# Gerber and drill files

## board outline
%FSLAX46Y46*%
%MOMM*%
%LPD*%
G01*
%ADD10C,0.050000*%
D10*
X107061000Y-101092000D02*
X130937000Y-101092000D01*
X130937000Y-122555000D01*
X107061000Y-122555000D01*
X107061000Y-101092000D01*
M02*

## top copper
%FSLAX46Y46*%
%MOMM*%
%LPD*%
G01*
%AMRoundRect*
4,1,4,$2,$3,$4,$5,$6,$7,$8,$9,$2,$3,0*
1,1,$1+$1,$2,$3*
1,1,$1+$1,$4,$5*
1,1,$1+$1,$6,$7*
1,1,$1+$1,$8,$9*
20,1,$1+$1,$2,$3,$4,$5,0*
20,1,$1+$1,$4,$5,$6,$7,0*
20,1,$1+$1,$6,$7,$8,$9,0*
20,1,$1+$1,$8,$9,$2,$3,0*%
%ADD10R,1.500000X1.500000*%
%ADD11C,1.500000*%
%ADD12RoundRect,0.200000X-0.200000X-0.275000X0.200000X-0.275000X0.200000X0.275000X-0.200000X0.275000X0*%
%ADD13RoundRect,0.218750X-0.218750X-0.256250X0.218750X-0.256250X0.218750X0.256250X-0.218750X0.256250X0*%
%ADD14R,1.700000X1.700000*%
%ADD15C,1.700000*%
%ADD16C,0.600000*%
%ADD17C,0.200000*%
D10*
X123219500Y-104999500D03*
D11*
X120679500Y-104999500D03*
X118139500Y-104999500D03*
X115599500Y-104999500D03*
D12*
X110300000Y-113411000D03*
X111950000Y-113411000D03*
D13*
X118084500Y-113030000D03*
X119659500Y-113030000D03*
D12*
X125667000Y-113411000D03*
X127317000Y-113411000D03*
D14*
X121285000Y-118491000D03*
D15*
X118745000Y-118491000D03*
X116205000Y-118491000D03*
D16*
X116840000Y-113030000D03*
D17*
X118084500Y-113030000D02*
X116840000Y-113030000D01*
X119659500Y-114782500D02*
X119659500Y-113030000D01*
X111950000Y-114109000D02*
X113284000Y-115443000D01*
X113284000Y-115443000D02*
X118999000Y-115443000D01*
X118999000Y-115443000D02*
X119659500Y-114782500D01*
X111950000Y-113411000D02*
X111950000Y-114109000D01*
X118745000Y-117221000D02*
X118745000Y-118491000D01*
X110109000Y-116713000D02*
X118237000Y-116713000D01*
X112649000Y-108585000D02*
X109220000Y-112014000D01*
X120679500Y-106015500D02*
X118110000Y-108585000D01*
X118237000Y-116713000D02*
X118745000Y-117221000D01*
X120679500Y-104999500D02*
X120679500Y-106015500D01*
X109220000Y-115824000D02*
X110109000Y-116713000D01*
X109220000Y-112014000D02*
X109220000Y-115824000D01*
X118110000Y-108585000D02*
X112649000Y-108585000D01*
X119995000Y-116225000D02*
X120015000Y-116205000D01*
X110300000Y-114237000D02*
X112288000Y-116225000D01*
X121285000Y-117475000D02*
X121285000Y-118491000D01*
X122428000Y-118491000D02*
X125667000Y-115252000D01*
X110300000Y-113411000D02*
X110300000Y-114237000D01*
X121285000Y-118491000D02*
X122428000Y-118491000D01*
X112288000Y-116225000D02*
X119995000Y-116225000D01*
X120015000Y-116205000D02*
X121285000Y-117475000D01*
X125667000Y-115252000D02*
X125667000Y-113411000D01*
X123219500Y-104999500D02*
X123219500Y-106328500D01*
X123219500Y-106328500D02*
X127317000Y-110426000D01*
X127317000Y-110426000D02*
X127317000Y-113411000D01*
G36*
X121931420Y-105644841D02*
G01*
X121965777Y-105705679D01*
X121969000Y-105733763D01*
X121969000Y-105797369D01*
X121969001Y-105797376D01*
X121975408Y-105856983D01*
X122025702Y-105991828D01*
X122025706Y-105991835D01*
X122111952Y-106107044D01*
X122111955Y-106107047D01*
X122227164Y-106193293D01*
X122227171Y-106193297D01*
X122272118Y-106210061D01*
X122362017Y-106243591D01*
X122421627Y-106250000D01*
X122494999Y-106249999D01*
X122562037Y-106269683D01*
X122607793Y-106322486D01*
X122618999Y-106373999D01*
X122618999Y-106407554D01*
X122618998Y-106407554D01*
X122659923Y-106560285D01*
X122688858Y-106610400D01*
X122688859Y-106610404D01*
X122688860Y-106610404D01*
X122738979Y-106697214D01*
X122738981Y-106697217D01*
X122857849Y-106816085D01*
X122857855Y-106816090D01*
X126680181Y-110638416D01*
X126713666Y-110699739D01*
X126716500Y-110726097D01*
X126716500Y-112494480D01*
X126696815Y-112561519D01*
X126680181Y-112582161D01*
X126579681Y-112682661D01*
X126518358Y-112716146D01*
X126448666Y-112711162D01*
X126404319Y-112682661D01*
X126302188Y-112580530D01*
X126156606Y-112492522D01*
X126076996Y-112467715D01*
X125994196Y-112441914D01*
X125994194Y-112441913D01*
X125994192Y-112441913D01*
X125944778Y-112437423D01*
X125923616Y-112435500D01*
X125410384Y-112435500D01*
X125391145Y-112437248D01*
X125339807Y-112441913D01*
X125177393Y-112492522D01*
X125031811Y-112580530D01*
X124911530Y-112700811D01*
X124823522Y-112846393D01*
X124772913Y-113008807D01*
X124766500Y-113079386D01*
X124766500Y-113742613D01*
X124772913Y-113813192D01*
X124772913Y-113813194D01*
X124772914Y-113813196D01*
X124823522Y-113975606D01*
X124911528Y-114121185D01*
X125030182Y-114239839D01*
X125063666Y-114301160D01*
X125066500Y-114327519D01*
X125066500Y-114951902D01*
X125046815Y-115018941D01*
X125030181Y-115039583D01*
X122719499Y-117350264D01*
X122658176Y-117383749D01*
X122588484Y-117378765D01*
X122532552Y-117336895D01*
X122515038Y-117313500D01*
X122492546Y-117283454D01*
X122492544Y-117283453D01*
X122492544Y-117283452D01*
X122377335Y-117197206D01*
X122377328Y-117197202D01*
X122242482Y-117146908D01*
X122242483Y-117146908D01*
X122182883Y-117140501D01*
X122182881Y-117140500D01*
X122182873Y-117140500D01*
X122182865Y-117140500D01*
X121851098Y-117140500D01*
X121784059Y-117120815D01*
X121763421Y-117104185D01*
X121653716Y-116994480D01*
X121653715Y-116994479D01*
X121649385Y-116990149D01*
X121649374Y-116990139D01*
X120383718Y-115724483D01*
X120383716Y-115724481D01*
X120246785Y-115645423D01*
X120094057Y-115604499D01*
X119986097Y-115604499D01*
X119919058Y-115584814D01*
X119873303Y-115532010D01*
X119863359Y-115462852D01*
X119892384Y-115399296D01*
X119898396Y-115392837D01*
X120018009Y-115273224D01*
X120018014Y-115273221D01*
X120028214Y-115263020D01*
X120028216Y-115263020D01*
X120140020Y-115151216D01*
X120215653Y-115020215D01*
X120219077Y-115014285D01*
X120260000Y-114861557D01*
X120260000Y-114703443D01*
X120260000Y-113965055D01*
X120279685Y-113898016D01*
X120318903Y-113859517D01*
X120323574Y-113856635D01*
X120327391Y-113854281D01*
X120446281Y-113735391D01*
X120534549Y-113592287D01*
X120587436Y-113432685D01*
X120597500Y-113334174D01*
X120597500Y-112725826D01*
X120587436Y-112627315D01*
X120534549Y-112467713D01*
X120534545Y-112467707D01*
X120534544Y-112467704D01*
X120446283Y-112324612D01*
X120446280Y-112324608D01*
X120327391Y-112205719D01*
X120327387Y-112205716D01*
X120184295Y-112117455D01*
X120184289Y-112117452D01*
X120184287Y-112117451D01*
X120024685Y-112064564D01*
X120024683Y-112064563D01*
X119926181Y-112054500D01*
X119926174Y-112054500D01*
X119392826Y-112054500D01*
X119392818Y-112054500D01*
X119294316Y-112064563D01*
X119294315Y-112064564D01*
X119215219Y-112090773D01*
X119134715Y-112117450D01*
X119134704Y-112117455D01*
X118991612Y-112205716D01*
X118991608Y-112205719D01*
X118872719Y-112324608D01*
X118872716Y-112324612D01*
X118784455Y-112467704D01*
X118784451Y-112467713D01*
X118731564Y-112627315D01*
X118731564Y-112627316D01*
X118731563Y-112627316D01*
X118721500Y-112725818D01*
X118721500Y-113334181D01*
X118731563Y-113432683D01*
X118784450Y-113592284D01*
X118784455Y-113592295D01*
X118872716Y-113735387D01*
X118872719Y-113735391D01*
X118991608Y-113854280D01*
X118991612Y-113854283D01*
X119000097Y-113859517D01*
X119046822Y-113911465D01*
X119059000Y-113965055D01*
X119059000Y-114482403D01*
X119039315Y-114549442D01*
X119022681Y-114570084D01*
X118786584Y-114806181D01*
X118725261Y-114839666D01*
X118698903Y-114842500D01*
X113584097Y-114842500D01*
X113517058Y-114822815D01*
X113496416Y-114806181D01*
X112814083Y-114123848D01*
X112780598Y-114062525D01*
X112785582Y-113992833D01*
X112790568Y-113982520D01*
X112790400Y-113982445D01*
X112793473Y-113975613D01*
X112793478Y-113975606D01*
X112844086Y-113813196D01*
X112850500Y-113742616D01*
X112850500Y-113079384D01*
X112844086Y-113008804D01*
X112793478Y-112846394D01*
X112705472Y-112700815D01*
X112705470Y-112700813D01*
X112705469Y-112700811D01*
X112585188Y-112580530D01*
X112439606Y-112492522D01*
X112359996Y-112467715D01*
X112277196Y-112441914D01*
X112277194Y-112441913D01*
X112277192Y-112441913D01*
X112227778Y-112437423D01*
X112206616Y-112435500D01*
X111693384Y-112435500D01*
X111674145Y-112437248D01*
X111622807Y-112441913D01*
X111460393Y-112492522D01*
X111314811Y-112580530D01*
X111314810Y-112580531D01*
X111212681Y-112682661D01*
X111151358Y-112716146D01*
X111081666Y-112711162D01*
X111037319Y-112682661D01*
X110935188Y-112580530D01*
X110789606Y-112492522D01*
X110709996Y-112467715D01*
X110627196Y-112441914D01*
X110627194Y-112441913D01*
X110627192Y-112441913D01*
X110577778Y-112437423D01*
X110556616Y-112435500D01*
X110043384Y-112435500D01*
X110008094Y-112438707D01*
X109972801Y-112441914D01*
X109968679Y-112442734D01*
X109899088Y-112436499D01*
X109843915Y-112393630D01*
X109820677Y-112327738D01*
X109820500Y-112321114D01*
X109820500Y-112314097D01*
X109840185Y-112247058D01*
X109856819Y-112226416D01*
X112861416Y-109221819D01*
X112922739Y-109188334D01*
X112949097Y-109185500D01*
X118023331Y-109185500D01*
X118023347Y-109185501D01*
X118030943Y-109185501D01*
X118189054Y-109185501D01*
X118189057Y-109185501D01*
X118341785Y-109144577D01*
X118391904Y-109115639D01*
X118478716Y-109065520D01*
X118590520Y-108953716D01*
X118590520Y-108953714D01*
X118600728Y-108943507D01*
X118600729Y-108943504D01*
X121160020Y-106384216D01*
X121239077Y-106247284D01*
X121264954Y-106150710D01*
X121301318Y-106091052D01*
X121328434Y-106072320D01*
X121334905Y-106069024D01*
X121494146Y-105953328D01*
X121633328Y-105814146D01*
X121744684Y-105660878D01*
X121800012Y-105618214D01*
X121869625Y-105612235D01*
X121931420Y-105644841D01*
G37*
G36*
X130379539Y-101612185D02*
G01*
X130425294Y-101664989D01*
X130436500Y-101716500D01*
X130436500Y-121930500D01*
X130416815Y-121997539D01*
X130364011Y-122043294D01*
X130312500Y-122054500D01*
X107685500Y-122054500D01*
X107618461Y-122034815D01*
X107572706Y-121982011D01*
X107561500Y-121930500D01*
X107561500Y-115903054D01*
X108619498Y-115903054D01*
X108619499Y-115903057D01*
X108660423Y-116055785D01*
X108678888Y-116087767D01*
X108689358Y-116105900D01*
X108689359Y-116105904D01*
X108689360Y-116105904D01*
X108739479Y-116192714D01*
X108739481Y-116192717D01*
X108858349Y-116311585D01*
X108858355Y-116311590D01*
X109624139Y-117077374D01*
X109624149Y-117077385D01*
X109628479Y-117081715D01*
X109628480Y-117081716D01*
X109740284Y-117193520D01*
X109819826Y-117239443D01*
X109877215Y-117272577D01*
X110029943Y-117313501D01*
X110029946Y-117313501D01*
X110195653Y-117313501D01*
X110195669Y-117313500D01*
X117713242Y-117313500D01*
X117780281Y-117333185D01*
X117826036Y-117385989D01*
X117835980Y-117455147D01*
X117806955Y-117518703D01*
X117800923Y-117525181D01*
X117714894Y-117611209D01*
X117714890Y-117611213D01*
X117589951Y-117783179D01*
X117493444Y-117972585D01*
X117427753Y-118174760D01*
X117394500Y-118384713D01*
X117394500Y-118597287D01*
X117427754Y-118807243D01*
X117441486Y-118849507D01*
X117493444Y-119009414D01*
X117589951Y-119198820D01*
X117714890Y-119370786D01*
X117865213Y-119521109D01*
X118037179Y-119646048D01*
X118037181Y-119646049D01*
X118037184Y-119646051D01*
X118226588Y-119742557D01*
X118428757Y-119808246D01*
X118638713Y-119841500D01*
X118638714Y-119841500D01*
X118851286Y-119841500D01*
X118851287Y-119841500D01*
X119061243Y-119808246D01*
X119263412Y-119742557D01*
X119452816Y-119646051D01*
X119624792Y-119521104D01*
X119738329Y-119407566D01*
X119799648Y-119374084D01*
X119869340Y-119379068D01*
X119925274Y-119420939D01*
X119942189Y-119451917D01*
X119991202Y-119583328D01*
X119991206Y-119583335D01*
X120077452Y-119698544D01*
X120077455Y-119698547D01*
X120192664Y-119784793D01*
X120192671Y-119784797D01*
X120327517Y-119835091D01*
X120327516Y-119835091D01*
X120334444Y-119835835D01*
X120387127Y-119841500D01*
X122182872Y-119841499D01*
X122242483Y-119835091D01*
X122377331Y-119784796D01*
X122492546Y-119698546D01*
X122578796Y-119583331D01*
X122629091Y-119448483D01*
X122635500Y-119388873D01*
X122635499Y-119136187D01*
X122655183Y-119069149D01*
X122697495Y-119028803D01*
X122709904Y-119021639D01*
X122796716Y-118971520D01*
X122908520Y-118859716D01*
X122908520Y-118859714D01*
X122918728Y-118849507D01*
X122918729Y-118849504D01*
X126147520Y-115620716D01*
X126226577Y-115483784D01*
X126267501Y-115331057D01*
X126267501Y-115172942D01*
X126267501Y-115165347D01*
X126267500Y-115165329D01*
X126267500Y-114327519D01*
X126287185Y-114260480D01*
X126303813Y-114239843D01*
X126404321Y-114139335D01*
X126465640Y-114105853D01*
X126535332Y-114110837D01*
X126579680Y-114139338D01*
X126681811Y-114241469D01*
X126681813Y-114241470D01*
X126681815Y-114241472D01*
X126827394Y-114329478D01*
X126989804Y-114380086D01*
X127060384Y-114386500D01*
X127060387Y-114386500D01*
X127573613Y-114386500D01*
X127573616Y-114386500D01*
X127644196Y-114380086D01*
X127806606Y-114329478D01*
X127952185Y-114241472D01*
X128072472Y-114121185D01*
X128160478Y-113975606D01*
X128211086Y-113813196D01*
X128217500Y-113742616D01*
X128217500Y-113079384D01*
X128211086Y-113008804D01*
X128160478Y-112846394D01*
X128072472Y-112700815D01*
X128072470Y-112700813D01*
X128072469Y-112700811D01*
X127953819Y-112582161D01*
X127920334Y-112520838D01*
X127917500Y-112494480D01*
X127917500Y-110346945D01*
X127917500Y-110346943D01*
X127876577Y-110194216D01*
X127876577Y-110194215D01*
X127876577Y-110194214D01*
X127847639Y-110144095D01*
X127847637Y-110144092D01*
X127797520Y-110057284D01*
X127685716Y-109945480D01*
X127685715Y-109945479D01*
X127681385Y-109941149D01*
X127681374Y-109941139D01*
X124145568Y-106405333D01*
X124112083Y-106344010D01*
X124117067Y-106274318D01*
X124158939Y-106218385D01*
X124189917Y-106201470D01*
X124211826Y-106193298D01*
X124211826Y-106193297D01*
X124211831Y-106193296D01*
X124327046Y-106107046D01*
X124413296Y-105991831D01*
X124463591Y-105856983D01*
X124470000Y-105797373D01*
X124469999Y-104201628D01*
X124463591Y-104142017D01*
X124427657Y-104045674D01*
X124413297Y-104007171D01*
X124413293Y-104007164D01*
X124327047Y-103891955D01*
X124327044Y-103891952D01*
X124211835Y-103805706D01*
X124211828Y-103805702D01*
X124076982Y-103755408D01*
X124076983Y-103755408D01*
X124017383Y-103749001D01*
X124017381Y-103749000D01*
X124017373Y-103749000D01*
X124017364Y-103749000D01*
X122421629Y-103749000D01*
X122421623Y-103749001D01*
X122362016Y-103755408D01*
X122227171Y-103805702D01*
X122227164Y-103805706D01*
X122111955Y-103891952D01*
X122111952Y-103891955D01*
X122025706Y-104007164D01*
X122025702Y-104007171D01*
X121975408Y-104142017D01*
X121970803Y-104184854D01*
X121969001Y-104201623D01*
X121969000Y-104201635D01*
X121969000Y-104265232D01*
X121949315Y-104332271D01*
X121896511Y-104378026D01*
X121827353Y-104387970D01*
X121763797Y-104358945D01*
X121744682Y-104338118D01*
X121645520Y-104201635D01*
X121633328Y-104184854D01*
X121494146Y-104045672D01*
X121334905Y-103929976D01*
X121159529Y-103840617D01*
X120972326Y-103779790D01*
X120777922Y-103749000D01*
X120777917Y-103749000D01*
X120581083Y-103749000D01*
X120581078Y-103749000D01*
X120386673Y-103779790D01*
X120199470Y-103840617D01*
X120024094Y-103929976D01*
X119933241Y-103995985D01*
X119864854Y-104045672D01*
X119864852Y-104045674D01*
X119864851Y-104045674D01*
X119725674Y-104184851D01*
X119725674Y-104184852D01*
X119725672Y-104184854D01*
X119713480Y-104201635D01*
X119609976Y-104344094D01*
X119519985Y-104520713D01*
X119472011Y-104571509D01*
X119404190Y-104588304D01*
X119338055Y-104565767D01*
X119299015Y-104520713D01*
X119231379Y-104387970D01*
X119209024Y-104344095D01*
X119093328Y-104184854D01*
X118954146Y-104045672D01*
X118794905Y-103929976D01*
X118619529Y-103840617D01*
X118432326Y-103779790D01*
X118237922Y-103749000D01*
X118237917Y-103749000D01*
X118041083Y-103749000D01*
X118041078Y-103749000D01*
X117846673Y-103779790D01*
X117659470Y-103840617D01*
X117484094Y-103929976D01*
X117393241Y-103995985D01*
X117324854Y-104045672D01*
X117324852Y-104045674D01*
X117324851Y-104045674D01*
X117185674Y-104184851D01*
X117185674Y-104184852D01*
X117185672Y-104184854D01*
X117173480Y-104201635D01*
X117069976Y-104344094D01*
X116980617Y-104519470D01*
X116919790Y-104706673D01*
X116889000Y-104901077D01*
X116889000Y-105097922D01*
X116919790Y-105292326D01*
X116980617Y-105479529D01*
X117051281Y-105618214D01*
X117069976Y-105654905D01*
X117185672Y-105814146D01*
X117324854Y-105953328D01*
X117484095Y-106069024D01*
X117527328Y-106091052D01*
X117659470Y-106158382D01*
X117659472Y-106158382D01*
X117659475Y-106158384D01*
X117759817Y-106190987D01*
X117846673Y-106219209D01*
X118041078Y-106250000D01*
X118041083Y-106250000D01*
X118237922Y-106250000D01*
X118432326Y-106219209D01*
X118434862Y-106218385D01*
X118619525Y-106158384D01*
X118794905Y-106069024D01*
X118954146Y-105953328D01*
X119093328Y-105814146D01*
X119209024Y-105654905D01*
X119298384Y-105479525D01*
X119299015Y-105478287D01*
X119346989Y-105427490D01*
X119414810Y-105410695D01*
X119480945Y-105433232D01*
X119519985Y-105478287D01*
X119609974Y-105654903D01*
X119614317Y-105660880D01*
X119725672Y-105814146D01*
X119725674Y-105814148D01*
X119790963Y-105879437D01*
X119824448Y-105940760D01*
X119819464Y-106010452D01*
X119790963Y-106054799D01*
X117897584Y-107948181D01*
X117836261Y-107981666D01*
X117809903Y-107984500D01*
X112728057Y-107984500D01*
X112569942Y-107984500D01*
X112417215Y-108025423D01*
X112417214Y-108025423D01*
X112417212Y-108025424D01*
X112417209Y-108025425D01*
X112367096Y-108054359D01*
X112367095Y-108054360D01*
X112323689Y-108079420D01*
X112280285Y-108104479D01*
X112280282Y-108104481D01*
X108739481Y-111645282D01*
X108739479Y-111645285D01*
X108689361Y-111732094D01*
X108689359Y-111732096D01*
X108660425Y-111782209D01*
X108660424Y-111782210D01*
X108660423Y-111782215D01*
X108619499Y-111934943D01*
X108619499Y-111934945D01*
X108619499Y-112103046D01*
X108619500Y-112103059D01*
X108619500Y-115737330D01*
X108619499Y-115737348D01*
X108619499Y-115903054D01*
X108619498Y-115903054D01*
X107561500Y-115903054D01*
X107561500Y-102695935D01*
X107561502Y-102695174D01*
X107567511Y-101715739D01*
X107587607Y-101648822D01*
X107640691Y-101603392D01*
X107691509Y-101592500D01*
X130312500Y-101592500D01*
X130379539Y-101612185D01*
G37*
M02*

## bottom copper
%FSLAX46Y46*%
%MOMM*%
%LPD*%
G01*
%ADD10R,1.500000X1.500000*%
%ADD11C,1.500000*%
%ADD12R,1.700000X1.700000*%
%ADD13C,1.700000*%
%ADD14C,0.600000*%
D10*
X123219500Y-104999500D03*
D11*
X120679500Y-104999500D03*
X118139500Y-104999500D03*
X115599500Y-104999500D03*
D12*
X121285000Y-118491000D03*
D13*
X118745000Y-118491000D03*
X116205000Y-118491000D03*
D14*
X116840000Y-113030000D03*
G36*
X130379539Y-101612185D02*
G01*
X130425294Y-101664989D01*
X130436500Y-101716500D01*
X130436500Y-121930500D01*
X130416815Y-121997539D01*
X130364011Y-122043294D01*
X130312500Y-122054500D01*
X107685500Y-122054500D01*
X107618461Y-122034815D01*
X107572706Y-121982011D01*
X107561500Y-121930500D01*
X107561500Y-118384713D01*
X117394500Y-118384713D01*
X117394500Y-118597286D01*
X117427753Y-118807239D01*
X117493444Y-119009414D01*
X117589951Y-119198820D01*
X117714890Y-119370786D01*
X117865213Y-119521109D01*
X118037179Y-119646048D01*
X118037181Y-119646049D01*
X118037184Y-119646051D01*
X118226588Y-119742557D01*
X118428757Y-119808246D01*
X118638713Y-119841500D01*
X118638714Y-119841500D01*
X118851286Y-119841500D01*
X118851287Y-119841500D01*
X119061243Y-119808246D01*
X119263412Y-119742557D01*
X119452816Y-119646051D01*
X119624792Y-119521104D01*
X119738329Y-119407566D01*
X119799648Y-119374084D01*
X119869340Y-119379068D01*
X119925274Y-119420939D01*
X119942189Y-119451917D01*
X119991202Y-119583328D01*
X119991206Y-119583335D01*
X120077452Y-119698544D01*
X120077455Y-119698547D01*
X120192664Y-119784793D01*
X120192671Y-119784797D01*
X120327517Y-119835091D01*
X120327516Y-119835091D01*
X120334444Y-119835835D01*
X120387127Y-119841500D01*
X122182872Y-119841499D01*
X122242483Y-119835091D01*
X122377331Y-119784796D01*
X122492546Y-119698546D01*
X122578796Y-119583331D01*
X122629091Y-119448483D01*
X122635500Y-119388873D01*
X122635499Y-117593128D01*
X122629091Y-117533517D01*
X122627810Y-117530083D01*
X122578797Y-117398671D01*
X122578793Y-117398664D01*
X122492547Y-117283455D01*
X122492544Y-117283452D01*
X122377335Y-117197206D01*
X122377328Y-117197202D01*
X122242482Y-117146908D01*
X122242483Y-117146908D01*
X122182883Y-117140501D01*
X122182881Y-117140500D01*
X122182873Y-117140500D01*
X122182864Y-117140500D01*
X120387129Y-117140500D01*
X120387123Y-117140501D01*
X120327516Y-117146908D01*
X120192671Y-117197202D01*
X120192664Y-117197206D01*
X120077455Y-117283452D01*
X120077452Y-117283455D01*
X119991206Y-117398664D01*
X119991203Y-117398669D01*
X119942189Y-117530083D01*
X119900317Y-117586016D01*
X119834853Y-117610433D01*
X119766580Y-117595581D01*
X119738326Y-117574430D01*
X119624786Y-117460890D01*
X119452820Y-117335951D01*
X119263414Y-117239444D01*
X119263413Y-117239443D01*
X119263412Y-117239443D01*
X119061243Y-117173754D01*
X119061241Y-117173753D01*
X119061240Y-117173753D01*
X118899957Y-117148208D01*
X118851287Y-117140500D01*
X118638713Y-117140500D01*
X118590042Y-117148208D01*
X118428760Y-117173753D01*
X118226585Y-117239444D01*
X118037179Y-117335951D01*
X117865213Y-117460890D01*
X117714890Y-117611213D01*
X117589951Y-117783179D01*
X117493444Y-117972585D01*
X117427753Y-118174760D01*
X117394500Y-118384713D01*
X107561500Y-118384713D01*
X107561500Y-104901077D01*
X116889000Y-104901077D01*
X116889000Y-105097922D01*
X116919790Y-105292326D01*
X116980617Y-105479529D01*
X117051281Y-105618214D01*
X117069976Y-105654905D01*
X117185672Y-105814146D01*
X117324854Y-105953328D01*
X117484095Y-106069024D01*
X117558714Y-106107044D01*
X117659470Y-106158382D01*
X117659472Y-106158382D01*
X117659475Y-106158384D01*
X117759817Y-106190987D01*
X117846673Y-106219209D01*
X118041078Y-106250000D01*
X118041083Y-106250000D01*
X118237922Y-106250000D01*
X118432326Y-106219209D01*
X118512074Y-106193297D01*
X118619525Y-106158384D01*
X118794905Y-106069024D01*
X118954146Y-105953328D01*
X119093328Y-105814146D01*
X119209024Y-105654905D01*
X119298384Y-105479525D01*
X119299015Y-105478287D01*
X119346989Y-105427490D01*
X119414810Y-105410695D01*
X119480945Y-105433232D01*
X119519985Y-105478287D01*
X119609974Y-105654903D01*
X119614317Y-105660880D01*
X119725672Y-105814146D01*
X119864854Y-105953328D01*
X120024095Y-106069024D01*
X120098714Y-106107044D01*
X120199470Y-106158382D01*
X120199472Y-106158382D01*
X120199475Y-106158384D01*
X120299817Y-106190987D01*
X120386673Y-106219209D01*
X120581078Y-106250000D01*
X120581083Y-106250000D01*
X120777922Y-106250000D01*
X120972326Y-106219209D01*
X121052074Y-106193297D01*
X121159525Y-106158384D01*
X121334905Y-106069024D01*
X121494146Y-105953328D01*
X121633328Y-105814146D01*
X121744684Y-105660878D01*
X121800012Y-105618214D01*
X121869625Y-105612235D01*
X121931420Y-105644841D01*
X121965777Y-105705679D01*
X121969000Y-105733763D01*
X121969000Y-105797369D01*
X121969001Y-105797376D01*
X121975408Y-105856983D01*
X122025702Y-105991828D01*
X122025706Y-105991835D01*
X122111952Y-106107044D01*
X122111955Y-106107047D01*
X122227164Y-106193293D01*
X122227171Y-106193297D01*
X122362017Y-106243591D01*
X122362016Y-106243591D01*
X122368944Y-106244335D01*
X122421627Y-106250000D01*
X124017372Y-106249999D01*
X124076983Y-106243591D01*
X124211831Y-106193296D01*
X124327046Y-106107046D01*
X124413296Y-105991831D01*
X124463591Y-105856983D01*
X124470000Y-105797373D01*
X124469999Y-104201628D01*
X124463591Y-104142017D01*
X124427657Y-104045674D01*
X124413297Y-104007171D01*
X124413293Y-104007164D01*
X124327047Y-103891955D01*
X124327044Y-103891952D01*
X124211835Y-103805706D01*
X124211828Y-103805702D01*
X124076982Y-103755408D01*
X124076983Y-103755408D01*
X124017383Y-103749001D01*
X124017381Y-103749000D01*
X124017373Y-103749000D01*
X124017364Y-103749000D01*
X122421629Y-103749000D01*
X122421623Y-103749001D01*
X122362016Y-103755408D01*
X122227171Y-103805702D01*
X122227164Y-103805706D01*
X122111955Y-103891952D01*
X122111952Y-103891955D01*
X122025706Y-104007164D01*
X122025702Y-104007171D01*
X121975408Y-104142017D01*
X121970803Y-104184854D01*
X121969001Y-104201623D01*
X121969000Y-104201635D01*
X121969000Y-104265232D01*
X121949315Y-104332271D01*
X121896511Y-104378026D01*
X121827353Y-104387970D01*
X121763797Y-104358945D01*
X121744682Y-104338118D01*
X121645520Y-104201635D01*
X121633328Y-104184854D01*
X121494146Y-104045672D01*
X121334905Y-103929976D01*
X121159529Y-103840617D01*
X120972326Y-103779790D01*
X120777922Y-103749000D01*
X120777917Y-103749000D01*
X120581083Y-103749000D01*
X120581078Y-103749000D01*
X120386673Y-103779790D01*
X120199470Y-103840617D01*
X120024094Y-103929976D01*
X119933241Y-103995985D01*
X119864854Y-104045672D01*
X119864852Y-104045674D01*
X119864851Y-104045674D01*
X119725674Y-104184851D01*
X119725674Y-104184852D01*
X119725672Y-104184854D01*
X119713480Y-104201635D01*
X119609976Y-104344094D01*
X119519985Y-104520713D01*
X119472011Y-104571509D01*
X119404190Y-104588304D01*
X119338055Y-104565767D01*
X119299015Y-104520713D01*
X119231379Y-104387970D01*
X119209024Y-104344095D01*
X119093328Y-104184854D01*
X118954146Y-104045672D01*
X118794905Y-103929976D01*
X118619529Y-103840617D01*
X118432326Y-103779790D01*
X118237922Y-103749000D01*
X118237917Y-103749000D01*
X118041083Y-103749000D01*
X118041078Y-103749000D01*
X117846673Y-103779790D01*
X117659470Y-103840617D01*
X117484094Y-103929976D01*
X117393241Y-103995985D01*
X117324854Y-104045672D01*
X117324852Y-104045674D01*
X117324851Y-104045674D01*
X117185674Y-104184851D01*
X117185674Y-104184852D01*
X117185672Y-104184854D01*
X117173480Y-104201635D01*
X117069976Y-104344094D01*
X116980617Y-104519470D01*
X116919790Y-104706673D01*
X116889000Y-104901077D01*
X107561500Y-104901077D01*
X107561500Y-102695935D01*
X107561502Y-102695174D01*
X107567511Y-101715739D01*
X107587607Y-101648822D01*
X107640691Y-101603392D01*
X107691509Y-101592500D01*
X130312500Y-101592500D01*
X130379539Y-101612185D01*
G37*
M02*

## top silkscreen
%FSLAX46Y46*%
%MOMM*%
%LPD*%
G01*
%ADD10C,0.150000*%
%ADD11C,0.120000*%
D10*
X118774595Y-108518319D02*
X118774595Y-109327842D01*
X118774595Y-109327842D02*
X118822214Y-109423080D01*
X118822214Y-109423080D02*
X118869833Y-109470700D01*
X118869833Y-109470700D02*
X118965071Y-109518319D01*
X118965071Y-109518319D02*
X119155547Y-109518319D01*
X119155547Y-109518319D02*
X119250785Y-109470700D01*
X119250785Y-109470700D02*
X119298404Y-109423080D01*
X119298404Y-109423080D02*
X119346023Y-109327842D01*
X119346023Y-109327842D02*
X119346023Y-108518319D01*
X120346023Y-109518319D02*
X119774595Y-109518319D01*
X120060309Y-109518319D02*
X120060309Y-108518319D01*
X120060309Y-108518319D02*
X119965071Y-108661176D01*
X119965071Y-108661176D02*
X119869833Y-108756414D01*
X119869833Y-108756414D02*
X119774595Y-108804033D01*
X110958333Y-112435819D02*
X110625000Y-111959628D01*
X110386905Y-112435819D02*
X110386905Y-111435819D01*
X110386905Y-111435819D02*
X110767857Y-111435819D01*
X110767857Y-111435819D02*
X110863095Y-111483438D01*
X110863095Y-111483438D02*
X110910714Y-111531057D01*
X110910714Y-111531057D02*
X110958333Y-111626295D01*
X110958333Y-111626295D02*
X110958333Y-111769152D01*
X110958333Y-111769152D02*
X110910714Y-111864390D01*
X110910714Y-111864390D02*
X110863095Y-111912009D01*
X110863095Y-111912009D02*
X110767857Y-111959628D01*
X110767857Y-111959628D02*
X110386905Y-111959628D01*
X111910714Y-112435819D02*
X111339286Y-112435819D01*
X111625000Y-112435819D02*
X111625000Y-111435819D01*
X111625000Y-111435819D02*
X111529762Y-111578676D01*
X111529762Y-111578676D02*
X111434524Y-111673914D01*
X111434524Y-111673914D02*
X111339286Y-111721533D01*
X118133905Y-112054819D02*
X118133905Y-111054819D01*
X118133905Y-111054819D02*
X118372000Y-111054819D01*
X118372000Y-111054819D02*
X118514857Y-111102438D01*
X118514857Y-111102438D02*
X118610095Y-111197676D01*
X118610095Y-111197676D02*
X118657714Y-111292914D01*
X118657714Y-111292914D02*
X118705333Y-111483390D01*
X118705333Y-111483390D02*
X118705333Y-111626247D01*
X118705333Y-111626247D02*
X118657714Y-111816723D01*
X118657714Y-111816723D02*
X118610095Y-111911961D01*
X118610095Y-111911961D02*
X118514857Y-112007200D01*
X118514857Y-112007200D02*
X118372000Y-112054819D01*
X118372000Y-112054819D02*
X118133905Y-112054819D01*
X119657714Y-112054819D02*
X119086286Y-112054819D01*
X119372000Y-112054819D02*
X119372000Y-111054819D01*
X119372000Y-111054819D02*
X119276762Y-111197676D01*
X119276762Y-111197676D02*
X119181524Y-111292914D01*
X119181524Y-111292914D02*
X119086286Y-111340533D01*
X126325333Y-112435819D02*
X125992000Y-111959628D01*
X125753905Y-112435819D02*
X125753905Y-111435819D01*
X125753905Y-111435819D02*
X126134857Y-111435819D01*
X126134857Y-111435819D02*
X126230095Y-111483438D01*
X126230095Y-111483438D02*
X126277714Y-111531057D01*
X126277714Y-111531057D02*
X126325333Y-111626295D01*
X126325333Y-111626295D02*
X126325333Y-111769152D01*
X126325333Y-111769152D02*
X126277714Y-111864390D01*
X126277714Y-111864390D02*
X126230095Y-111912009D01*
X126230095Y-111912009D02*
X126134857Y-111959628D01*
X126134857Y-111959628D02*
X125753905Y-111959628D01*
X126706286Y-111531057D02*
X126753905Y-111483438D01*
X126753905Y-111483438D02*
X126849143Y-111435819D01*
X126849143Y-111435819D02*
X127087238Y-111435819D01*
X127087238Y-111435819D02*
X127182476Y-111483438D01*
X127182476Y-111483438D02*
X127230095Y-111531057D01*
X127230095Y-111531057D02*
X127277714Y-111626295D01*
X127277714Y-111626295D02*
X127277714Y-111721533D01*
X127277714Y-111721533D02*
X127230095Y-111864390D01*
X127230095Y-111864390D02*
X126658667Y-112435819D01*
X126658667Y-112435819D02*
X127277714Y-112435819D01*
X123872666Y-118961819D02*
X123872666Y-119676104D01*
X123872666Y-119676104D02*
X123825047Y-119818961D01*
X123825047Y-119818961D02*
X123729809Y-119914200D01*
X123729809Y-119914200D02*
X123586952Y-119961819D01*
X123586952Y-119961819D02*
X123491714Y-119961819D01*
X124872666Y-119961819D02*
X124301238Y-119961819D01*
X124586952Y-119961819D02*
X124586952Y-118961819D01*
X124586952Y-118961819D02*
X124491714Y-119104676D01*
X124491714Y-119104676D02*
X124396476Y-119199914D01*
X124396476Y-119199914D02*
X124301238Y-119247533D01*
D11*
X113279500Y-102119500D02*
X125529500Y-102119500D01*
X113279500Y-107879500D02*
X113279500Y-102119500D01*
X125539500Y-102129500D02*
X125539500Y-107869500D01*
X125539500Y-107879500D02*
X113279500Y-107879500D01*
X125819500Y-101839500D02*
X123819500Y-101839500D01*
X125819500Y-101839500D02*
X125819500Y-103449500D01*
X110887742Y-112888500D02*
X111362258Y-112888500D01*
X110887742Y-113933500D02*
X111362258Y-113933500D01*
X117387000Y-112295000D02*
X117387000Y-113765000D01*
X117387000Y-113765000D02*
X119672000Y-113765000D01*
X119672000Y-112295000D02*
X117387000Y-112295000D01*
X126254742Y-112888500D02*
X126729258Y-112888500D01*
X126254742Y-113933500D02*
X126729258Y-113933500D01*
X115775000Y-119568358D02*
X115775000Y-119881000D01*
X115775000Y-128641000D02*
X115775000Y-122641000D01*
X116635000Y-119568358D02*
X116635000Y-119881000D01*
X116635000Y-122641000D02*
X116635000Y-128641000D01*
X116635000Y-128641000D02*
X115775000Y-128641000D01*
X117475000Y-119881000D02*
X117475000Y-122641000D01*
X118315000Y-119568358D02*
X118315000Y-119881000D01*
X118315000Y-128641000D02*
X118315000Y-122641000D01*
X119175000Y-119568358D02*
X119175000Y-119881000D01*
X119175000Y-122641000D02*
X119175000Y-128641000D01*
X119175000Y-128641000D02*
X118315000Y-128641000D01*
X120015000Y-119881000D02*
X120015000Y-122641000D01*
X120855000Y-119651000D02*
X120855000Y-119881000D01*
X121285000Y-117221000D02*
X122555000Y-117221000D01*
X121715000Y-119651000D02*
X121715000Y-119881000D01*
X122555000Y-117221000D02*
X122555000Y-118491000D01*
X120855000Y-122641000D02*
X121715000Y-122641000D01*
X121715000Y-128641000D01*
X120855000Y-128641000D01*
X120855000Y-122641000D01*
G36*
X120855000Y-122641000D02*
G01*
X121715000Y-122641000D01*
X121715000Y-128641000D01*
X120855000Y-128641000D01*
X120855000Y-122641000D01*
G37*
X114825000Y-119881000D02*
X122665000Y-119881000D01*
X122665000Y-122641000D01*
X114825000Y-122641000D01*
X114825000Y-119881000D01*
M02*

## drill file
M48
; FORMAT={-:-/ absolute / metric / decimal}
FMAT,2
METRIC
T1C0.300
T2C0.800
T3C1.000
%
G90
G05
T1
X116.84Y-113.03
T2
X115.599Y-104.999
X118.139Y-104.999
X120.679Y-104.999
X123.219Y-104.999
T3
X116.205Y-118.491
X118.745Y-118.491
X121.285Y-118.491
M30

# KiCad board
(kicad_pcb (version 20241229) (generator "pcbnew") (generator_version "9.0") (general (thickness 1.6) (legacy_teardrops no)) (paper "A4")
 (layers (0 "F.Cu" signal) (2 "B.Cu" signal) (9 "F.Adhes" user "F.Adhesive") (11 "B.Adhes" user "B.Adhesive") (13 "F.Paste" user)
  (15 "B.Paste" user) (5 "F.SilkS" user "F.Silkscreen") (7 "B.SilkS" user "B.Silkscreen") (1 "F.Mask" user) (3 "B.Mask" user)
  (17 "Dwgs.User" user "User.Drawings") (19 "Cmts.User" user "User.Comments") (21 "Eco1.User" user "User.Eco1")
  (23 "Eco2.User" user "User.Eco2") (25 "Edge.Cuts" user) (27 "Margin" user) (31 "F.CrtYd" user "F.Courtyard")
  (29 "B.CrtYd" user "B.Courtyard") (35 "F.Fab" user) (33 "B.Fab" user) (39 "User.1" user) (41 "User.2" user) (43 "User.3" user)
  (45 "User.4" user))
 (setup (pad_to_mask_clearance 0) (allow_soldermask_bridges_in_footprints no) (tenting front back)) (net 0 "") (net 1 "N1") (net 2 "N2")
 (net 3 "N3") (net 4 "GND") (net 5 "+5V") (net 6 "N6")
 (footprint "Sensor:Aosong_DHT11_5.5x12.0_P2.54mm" (layer "F.Cu") (at 123.2195 104.9995 -90)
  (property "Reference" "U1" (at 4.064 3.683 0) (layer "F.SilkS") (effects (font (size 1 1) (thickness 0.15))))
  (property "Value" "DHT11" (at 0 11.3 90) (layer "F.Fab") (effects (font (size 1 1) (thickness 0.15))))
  (fp_line (start -2.88 9.94) (end -2.88 -2.31) (stroke (width 0.12) (type solid)) (layer "F.SilkS"))
  (fp_line (start 2.88 9.94) (end -2.88 9.94) (stroke (width 0.12) (type solid)) (layer "F.SilkS"))
  (fp_line (start -2.87 -2.32) (end 2.87 -2.32) (stroke (width 0.12) (type solid)) (layer "F.SilkS"))
  (fp_line (start 2.88 -2.32) (end 2.88 9.94) (stroke (width 0.12) (type solid)) (layer "F.SilkS"))
  (fp_line (start -3.16 -2.6) (end -3.16 -0.6) (stroke (width 0.12) (type solid)) (layer "F.SilkS"))
  (fp_line (start -3.16 -2.6) (end -1.55 -2.6) (stroke (width 0.12) (type solid)) (layer "F.SilkS"))
  (pad "1" thru_hole rect (at 0 0 270) (size 1.5 1.5) (drill 0.8) (layers "*.Cu" "*.Mask") (remove_unused_layers no) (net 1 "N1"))
  (pad "2" thru_hole circle (at 0 2.54 270) (size 1.5 1.5) (drill 0.8) (layers "*.Cu" "*.Mask") (remove_unused_layers no) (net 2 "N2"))
  (pad "3" thru_hole circle (at 0 5.08 270) (size 1.5 1.5) (drill 0.8) (layers "*.Cu" "*.Mask") (remove_unused_layers no) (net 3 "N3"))
  (pad "4" thru_hole circle (at 0 7.62 270) (size 1.5 1.5) (drill 0.8) (layers "*.Cu" "*.Mask") (remove_unused_layers no) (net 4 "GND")))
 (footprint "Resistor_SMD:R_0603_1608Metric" (layer "F.Cu") (at 111.125 113.411)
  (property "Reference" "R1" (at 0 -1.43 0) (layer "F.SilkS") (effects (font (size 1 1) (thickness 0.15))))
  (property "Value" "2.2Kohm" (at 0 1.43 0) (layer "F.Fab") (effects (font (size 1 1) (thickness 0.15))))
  (fp_line (start -0.237258 -0.5225) (end 0.237258 -0.5225) (stroke (width 0.12) (type solid)) (layer "F.SilkS"))
  (fp_line (start -0.237258 0.5225) (end 0.237258 0.5225) (stroke (width 0.12) (type solid)) (layer "F.SilkS"))
  (pad "1" smd roundrect (at -0.825 0) (size 0.8 0.95) (layers "F.Cu" "F.Mask" "F.Paste") (roundrect_rratio 0.25) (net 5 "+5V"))
  (pad "2" smd roundrect (at 0.825 0) (size 0.8 0.95) (layers "F.Cu" "F.Mask" "F.Paste") (roundrect_rratio 0.25) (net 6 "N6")))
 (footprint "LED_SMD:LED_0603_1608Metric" (layer "F.Cu") (at 118.872 113.03)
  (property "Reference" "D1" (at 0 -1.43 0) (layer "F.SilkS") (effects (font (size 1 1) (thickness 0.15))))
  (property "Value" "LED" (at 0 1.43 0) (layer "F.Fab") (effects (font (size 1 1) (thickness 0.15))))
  (fp_line (start -1.485 -0.735) (end -1.485 0.735) (stroke (width 0.12) (type solid)) (layer "F.SilkS"))
  (fp_line (start -1.485 0.735) (end 0.8 0.735) (stroke (width 0.12) (type solid)) (layer "F.SilkS"))
  (fp_line (start 0.8 -0.735) (end -1.485 -0.735) (stroke (width 0.12) (type solid)) (layer "F.SilkS"))
  (pad "1" smd roundrect (at -0.7875 0) (size 0.875 0.95) (layers "F.Cu" "F.Mask" "F.Paste") (roundrect_rratio 0.25) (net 4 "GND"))
  (pad "2" smd roundrect (at 0.7875 0) (size 0.875 0.95) (layers "F.Cu" "F.Mask" "F.Paste") (roundrect_rratio 0.25) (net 6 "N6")))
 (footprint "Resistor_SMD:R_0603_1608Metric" (layer "F.Cu") (at 126.492 113.411)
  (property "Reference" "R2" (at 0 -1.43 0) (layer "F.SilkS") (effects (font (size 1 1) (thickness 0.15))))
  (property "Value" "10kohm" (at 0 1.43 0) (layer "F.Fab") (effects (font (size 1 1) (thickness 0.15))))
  (fp_line (start -0.237258 -0.5225) (end 0.237258 -0.5225) (stroke (width 0.12) (type solid)) (layer "F.SilkS"))
  (fp_line (start -0.237258 0.5225) (end 0.237258 0.5225) (stroke (width 0.12) (type solid)) (layer "F.SilkS"))
  (pad "1" smd roundrect (at -0.825 0) (size 0.8 0.95) (layers "F.Cu" "F.Mask" "F.Paste") (roundrect_rratio 0.25) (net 5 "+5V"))
  (pad "2" smd roundrect (at 0.825 0) (size 0.8 0.95) (layers "F.Cu" "F.Mask" "F.Paste") (roundrect_rratio 0.25) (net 1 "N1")))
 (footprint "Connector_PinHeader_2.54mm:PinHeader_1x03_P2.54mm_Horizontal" (layer "F.Cu") (at 121.285 118.491 -90)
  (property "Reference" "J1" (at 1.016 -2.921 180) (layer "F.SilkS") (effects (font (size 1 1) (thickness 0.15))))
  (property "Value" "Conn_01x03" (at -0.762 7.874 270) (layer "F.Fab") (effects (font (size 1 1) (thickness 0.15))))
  (fp_line (start 1.077358 5.51) (end 1.39 5.51) (stroke (width 0.12) (type solid)) (layer "F.SilkS"))
  (fp_line (start 10.15 5.51) (end 4.15 5.51) (stroke (width 0.12) (type solid)) (layer "F.SilkS"))
  (fp_line (start 1.077358 4.65) (end 1.39 4.65) (stroke (width 0.12) (type solid)) (layer "F.SilkS"))
  (fp_line (start 4.15 4.65) (end 10.15 4.65) (stroke (width 0.12) (type solid)) (layer "F.SilkS"))
  (fp_line (start 10.15 4.65) (end 10.15 5.51) (stroke (width 0.12) (type solid)) (layer "F.SilkS"))
  (fp_line (start 1.39 3.81) (end 4.15 3.81) (stroke (width 0.12) (type solid)) (layer "F.SilkS"))
  (fp_line (start 1.077358 2.97) (end 1.39 2.97) (stroke (width 0.12) (type solid)) (layer "F.SilkS"))
  (fp_line (start 10.15 2.97) (end 4.15 2.97) (stroke (width 0.12) (type solid)) (layer "F.SilkS"))
  (fp_line (start 1.077358 2.11) (end 1.39 2.11) (stroke (width 0.12) (type solid)) (layer "F.SilkS"))
  (fp_line (start 4.15 2.11) (end 10.15 2.11) (stroke (width 0.12) (type solid)) (layer "F.SilkS"))
  (fp_line (start 10.15 2.11) (end 10.15 2.97) (stroke (width 0.12) (type solid)) (layer "F.SilkS"))
  (fp_line (start 1.39 1.27) (end 4.15 1.27) (stroke (width 0.12) (type solid)) (layer "F.SilkS"))
  (fp_line (start 1.16 0.43) (end 1.39 0.43) (stroke (width 0.12) (type solid)) (layer "F.SilkS"))
  (fp_line (start -1.27 0) (end -1.27 -1.27) (stroke (width 0.12) (type solid)) (layer "F.SilkS"))
  (fp_line (start 1.16 -0.43) (end 1.39 -0.43) (stroke (width 0.12) (type solid)) (layer "F.SilkS"))
  (fp_line (start -1.27 -1.27) (end 0 -1.27) (stroke (width 0.12) (type solid)) (layer "F.SilkS"))
  (fp_rect (start 4.15 -0.43) (end 10.15 0.43) (stroke (width 0.12) (type solid)) (fill yes) (layer "F.SilkS"))
  (fp_rect (start 1.39 -1.38) (end 4.15 6.46) (stroke (width 0.12) (type solid)) (fill no) (layer "F.SilkS"))
  (pad "1" thru_hole rect (at 0 0 270) (size 1.7 1.7) (drill 1) (layers "*.Cu" "*.Mask") (remove_unused_layers no) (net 5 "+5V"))
  (pad "2" thru_hole circle (at 0 2.54 270) (size 1.7 1.7) (drill 1) (layers "*.Cu" "*.Mask") (remove_unused_layers no) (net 2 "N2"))
  (pad "3" thru_hole circle (at 0 5.08 270) (size 1.7 1.7) (drill 1) (layers "*.Cu" "*.Mask") (remove_unused_layers no) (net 4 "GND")))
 (gr_rect (start 107.061 101.092) (end 130.937 122.555) (stroke (width 0.05) (type default)) (fill no) (layer "Edge.Cuts"))
 (segment (start 118.0845 113.03) (end 116.84 113.03) (width 0.2) (layer "F.Cu") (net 4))
 (via (at 116.84 113.03) (size 0.6) (drill 0.3) (layers "F.Cu" "B.Cu") (free yes) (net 4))
 (segment (start 119.6595 114.7825) (end 119.6595 113.03) (width 0.2) (layer "F.Cu") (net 6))
 (segment (start 111.95 114.109) (end 113.284 115.443) (width 0.2) (layer "F.Cu") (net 6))
 (segment (start 113.284 115.443) (end 118.999 115.443) (width 0.2) (layer "F.Cu") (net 6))
 (segment (start 118.999 115.443) (end 119.6595 114.7825) (width 0.2) (layer "F.Cu") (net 6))
 (segment (start 111.95 113.411) (end 111.95 114.109) (width 0.2) (layer "F.Cu") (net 6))
 (segment (start 118.745 117.221) (end 118.745 118.491) (width 0.2) (layer "F.Cu") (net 2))
 (segment (start 110.109 116.713) (end 118.237 116.713) (width 0.2) (layer "F.Cu") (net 2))
 (segment (start 112.649 108.585) (end 109.22 112.014) (width 0.2) (layer "F.Cu") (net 2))
 (segment (start 120.6795 106.0155) (end 118.11 108.585) (width 0.2) (layer "F.Cu") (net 2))
 (segment (start 118.237 116.713) (end 118.745 117.221) (width 0.2) (layer "F.Cu") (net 2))
 (segment (start 120.6795 104.9995) (end 120.6795 106.0155) (width 0.2) (layer "F.Cu") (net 2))
 (segment (start 109.22 115.824) (end 110.109 116.713) (width 0.2) (layer "F.Cu") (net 2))
 (segment (start 109.22 112.014) (end 109.22 115.824) (width 0.2) (layer "F.Cu") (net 2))
 (segment (start 118.11 108.585) (end 112.649 108.585) (width 0.2) (layer "F.Cu") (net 2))
 (segment (start 119.995 116.225) (end 120.015 116.205) (width 0.2) (layer "F.Cu") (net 5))
 (segment (start 110.3 114.237) (end 112.288 116.225) (width 0.2) (layer "F.Cu") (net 5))
 (segment (start 121.285 117.475) (end 121.285 118.491) (width 0.2) (layer "F.Cu") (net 5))
 (segment (start 122.428 118.491) (end 125.667 115.252) (width 0.2) (layer "F.Cu") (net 5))
 (segment (start 110.3 113.411) (end 110.3 114.237) (width 0.2) (layer "F.Cu") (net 5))
 (segment (start 121.285 118.491) (end 122.428 118.491) (width 0.2) (layer "F.Cu") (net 5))
 (segment (start 112.288 116.225) (end 119.995 116.225) (width 0.2) (layer "F.Cu") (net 5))
 (segment (start 120.015 116.205) (end 121.285 117.475) (width 0.2) (layer "F.Cu") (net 5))
 (segment (start 125.667 115.252) (end 125.667 113.411) (width 0.2) (layer "F.Cu") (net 5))
 (segment (start 123.2195 104.9995) (end 123.2195 106.3285) (width 0.2) (layer "F.Cu") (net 1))
 (segment (start 123.2195 106.3285) (end 127.317 110.426) (width 0.2) (layer "F.Cu") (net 1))
 (segment (start 127.317 110.426) (end 127.317 113.411) (width 0.2) (layer "F.Cu") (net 1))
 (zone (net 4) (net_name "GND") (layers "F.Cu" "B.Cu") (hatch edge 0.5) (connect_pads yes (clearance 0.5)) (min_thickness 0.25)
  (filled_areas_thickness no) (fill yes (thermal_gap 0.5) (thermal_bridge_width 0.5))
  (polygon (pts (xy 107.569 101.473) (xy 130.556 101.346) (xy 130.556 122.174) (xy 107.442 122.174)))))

